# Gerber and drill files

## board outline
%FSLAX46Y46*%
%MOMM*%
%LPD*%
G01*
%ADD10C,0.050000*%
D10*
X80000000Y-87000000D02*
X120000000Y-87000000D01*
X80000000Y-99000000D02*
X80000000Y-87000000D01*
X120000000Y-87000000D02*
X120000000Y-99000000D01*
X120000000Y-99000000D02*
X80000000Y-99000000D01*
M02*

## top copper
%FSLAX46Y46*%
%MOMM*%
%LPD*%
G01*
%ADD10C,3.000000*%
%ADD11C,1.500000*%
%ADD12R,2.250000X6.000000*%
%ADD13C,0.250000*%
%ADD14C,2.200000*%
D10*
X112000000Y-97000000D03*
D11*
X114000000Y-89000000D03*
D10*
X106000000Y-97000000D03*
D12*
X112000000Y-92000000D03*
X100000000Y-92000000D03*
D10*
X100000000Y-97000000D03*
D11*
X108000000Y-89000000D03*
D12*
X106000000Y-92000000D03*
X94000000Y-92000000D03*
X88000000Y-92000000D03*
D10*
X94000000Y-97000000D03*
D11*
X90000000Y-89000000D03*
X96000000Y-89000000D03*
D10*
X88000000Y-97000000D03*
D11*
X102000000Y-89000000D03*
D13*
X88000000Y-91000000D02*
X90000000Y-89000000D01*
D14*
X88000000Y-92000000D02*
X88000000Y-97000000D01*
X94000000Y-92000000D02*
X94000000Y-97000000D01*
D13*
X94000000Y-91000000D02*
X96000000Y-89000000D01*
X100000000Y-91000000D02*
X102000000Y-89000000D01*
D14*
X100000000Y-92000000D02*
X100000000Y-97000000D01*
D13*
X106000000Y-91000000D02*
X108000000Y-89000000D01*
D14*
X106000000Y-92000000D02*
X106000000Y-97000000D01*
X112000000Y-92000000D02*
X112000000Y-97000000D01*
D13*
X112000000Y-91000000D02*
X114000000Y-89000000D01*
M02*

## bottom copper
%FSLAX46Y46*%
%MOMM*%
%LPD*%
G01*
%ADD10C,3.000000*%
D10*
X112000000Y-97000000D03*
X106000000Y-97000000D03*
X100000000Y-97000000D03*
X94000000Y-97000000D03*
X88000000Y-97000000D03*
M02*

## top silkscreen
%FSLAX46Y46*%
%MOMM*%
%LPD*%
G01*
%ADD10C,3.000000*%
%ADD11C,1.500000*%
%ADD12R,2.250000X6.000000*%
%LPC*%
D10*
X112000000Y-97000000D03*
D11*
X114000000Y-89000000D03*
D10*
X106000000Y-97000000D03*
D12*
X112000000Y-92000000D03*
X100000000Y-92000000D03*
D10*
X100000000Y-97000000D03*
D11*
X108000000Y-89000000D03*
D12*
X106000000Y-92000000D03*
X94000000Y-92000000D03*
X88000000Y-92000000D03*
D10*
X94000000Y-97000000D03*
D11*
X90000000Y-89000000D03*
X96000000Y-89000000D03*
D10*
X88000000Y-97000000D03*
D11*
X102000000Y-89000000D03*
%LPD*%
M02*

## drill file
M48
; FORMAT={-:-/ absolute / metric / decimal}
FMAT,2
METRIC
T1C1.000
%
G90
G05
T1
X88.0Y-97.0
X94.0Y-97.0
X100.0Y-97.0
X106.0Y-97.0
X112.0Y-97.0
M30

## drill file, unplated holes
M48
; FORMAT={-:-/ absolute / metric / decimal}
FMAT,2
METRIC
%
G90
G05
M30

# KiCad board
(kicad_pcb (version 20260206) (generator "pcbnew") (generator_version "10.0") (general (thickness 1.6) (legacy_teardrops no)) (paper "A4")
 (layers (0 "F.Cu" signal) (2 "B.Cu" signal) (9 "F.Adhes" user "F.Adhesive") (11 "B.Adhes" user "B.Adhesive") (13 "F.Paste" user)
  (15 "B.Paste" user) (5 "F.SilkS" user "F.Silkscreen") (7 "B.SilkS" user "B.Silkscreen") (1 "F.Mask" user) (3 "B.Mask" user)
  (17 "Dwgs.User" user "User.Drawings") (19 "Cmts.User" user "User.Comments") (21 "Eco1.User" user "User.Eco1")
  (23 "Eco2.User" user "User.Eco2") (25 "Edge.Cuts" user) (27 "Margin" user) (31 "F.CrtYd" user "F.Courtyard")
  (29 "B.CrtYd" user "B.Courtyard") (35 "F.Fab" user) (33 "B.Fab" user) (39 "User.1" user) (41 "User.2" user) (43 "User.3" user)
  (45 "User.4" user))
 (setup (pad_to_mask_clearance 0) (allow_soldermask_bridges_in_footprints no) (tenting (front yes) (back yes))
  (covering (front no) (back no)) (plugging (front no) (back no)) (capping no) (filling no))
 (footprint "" (layer "F.Cu") (at 112 97)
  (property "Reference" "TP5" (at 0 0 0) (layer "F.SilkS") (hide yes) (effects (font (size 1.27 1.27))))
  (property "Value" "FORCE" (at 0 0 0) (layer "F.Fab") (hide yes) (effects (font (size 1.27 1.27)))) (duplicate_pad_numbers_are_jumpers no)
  (pad "1" thru_hole circle (at 0 0) (size 3 3) (drill 1) (layers "*.Cu" "*.Mask") (remove_unused_layers no) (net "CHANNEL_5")))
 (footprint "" (layer "F.Cu") (at 114 89)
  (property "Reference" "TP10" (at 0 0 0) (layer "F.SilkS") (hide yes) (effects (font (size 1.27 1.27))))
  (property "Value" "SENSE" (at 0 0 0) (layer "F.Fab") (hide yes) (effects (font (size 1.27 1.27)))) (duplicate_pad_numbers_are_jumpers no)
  (pad "1" smd circle (at 0 0) (size 1.5 1.5) (layers "F.Cu" "F.Mask") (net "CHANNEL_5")))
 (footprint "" (layer "F.Cu") (at 106 97)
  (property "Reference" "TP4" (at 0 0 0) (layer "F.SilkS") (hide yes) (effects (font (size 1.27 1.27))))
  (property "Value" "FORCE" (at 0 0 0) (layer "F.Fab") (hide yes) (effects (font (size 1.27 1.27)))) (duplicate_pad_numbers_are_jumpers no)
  (pad "1" thru_hole circle (at 0 0) (size 3 3) (drill 1) (layers "*.Cu" "*.Mask") (remove_unused_layers no) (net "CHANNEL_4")))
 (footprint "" (layer "F.Cu") (at 112 92)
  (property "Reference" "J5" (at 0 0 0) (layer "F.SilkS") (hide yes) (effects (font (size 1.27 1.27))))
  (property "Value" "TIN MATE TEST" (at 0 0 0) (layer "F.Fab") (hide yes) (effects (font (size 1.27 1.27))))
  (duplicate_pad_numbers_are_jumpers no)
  (pad "1" smd rect (at 0 0) (size 2.25 6) (layers "F.Cu" "F.Mask") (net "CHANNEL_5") (thermal_bridge_angle 45)))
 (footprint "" (layer "F.Cu") (at 100 92)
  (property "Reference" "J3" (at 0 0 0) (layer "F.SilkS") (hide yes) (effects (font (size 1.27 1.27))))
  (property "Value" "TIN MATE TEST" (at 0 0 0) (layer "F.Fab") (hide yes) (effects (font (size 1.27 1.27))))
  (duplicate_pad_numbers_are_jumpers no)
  (pad "1" smd rect (at 0 0) (size 2.25 6) (layers "F.Cu" "F.Mask") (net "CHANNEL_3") (thermal_bridge_angle 45)))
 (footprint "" (layer "F.Cu") (at 100 97)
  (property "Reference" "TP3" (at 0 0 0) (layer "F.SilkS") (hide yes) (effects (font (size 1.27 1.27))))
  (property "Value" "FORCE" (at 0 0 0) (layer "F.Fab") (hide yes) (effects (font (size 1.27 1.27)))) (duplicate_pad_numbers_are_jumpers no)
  (pad "1" thru_hole circle (at 0 0) (size 3 3) (drill 1) (layers "*.Cu" "*.Mask") (remove_unused_layers no) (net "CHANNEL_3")))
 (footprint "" (layer "F.Cu") (at 108 89)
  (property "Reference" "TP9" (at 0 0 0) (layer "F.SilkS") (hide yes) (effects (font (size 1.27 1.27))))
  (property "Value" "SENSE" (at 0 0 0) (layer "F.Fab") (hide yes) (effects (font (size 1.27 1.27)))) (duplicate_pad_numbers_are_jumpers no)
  (pad "1" smd circle (at 0 0) (size 1.5 1.5) (layers "F.Cu" "F.Mask") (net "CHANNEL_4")))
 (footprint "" (layer "F.Cu") (at 106 92)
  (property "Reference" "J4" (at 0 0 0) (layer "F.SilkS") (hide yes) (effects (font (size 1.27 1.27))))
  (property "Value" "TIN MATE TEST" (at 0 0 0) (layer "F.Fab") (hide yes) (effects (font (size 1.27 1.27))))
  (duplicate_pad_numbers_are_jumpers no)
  (pad "1" smd rect (at 0 0) (size 2.25 6) (layers "F.Cu" "F.Mask") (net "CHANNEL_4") (thermal_bridge_angle 45)))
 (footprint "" (layer "F.Cu") (at 94 92)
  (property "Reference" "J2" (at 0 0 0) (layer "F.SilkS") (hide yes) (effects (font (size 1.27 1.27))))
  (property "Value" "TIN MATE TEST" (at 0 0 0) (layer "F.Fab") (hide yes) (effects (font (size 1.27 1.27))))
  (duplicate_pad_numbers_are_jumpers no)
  (pad "1" smd rect (at 0 0) (size 2.25 6) (layers "F.Cu" "F.Mask") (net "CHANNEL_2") (thermal_bridge_angle 45)))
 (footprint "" (layer "F.Cu") (at 88 92)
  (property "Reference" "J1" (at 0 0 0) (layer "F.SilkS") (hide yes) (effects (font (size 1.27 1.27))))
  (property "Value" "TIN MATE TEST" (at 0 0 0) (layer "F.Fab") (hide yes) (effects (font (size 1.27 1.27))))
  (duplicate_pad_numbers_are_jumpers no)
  (pad "1" smd rect (at 0 0) (size 2.25 6) (layers "F.Cu" "F.Mask") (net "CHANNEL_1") (thermal_bridge_angle 45)))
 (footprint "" (layer "F.Cu") (at 94 97)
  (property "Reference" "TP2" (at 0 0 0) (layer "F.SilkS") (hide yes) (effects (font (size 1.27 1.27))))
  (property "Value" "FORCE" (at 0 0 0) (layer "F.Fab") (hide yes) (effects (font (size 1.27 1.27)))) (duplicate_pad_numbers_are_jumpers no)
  (pad "1" thru_hole circle (at 0 0) (size 3 3) (drill 1) (layers "*.Cu" "*.Mask") (remove_unused_layers no) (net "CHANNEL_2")))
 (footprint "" (layer "F.Cu") (at 90 89)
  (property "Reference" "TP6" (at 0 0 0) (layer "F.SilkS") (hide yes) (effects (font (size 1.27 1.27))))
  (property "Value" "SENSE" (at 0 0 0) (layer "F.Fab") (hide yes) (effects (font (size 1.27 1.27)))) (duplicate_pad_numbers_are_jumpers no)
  (pad "1" smd circle (at 0 0) (size 1.5 1.5) (layers "F.Cu" "F.Mask") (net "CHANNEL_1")))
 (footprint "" (layer "F.Cu") (at 96 89)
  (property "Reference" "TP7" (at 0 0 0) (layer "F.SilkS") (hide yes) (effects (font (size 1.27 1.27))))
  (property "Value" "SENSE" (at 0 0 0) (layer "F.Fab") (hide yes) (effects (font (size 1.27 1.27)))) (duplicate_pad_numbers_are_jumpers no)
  (pad "1" smd circle (at 0 0) (size 1.5 1.5) (layers "F.Cu" "F.Mask") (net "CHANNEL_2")))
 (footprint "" (layer "F.Cu") (at 88 97)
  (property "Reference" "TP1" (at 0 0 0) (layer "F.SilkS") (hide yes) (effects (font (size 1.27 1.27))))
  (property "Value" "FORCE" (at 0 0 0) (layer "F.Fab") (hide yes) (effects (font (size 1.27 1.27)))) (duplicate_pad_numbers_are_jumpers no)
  (pad "1" thru_hole circle (at 0 0) (size 3 3) (drill 1) (layers "*.Cu" "*.Mask") (remove_unused_layers no) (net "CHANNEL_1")))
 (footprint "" (layer "F.Cu") (at 102 89)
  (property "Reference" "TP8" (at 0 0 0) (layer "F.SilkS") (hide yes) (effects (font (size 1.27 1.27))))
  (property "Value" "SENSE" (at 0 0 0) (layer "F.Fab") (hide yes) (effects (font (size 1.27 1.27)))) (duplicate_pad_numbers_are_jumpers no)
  (pad "1" smd circle (at 0 0) (size 1.5 1.5) (layers "F.Cu" "F.Mask") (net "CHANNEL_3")))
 (gr_line (start 80 87) (end 120 87) (stroke (width 0.05) (type default)) (layer "Edge.Cuts"))
 (gr_line (start 80 99) (end 80 87) (stroke (width 0.05) (type default)) (layer "Edge.Cuts"))
 (gr_line (start 120 87) (end 120 99) (stroke (width 0.05) (type default)) (layer "Edge.Cuts"))
 (gr_line (start 120 99) (end 80 99) (stroke (width 0.05) (type default)) (layer "Edge.Cuts"))
 (segment (start 88 91) (end 90 89) (width 0.25) (layer "F.Cu") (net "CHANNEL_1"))
 (segment (start 88 92) (end 88 97) (width 2.2) (layer "F.Cu") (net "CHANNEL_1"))
 (segment (start 94 92) (end 94 97) (width 2.2) (layer "F.Cu") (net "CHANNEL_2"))
 (segment (start 94 91) (end 96 89) (width 0.25) (layer "F.Cu") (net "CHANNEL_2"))
 (segment (start 100 91) (end 102 89) (width 0.25) (layer "F.Cu") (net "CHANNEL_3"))
 (segment (start 100 92) (end 100 97) (width 2.2) (layer "F.Cu") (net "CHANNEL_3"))
 (segment (start 106 91) (end 108 89) (width 0.25) (layer "F.Cu") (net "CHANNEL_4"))
 (segment (start 106 92) (end 106 97) (width 2.2) (layer "F.Cu") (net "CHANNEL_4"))
 (segment (start 112 92) (end 112 97) (width 2.2) (layer "F.Cu") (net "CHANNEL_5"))
 (segment (start 112 91) (end 114 89) (width 0.25) (layer "F.Cu") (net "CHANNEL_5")))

